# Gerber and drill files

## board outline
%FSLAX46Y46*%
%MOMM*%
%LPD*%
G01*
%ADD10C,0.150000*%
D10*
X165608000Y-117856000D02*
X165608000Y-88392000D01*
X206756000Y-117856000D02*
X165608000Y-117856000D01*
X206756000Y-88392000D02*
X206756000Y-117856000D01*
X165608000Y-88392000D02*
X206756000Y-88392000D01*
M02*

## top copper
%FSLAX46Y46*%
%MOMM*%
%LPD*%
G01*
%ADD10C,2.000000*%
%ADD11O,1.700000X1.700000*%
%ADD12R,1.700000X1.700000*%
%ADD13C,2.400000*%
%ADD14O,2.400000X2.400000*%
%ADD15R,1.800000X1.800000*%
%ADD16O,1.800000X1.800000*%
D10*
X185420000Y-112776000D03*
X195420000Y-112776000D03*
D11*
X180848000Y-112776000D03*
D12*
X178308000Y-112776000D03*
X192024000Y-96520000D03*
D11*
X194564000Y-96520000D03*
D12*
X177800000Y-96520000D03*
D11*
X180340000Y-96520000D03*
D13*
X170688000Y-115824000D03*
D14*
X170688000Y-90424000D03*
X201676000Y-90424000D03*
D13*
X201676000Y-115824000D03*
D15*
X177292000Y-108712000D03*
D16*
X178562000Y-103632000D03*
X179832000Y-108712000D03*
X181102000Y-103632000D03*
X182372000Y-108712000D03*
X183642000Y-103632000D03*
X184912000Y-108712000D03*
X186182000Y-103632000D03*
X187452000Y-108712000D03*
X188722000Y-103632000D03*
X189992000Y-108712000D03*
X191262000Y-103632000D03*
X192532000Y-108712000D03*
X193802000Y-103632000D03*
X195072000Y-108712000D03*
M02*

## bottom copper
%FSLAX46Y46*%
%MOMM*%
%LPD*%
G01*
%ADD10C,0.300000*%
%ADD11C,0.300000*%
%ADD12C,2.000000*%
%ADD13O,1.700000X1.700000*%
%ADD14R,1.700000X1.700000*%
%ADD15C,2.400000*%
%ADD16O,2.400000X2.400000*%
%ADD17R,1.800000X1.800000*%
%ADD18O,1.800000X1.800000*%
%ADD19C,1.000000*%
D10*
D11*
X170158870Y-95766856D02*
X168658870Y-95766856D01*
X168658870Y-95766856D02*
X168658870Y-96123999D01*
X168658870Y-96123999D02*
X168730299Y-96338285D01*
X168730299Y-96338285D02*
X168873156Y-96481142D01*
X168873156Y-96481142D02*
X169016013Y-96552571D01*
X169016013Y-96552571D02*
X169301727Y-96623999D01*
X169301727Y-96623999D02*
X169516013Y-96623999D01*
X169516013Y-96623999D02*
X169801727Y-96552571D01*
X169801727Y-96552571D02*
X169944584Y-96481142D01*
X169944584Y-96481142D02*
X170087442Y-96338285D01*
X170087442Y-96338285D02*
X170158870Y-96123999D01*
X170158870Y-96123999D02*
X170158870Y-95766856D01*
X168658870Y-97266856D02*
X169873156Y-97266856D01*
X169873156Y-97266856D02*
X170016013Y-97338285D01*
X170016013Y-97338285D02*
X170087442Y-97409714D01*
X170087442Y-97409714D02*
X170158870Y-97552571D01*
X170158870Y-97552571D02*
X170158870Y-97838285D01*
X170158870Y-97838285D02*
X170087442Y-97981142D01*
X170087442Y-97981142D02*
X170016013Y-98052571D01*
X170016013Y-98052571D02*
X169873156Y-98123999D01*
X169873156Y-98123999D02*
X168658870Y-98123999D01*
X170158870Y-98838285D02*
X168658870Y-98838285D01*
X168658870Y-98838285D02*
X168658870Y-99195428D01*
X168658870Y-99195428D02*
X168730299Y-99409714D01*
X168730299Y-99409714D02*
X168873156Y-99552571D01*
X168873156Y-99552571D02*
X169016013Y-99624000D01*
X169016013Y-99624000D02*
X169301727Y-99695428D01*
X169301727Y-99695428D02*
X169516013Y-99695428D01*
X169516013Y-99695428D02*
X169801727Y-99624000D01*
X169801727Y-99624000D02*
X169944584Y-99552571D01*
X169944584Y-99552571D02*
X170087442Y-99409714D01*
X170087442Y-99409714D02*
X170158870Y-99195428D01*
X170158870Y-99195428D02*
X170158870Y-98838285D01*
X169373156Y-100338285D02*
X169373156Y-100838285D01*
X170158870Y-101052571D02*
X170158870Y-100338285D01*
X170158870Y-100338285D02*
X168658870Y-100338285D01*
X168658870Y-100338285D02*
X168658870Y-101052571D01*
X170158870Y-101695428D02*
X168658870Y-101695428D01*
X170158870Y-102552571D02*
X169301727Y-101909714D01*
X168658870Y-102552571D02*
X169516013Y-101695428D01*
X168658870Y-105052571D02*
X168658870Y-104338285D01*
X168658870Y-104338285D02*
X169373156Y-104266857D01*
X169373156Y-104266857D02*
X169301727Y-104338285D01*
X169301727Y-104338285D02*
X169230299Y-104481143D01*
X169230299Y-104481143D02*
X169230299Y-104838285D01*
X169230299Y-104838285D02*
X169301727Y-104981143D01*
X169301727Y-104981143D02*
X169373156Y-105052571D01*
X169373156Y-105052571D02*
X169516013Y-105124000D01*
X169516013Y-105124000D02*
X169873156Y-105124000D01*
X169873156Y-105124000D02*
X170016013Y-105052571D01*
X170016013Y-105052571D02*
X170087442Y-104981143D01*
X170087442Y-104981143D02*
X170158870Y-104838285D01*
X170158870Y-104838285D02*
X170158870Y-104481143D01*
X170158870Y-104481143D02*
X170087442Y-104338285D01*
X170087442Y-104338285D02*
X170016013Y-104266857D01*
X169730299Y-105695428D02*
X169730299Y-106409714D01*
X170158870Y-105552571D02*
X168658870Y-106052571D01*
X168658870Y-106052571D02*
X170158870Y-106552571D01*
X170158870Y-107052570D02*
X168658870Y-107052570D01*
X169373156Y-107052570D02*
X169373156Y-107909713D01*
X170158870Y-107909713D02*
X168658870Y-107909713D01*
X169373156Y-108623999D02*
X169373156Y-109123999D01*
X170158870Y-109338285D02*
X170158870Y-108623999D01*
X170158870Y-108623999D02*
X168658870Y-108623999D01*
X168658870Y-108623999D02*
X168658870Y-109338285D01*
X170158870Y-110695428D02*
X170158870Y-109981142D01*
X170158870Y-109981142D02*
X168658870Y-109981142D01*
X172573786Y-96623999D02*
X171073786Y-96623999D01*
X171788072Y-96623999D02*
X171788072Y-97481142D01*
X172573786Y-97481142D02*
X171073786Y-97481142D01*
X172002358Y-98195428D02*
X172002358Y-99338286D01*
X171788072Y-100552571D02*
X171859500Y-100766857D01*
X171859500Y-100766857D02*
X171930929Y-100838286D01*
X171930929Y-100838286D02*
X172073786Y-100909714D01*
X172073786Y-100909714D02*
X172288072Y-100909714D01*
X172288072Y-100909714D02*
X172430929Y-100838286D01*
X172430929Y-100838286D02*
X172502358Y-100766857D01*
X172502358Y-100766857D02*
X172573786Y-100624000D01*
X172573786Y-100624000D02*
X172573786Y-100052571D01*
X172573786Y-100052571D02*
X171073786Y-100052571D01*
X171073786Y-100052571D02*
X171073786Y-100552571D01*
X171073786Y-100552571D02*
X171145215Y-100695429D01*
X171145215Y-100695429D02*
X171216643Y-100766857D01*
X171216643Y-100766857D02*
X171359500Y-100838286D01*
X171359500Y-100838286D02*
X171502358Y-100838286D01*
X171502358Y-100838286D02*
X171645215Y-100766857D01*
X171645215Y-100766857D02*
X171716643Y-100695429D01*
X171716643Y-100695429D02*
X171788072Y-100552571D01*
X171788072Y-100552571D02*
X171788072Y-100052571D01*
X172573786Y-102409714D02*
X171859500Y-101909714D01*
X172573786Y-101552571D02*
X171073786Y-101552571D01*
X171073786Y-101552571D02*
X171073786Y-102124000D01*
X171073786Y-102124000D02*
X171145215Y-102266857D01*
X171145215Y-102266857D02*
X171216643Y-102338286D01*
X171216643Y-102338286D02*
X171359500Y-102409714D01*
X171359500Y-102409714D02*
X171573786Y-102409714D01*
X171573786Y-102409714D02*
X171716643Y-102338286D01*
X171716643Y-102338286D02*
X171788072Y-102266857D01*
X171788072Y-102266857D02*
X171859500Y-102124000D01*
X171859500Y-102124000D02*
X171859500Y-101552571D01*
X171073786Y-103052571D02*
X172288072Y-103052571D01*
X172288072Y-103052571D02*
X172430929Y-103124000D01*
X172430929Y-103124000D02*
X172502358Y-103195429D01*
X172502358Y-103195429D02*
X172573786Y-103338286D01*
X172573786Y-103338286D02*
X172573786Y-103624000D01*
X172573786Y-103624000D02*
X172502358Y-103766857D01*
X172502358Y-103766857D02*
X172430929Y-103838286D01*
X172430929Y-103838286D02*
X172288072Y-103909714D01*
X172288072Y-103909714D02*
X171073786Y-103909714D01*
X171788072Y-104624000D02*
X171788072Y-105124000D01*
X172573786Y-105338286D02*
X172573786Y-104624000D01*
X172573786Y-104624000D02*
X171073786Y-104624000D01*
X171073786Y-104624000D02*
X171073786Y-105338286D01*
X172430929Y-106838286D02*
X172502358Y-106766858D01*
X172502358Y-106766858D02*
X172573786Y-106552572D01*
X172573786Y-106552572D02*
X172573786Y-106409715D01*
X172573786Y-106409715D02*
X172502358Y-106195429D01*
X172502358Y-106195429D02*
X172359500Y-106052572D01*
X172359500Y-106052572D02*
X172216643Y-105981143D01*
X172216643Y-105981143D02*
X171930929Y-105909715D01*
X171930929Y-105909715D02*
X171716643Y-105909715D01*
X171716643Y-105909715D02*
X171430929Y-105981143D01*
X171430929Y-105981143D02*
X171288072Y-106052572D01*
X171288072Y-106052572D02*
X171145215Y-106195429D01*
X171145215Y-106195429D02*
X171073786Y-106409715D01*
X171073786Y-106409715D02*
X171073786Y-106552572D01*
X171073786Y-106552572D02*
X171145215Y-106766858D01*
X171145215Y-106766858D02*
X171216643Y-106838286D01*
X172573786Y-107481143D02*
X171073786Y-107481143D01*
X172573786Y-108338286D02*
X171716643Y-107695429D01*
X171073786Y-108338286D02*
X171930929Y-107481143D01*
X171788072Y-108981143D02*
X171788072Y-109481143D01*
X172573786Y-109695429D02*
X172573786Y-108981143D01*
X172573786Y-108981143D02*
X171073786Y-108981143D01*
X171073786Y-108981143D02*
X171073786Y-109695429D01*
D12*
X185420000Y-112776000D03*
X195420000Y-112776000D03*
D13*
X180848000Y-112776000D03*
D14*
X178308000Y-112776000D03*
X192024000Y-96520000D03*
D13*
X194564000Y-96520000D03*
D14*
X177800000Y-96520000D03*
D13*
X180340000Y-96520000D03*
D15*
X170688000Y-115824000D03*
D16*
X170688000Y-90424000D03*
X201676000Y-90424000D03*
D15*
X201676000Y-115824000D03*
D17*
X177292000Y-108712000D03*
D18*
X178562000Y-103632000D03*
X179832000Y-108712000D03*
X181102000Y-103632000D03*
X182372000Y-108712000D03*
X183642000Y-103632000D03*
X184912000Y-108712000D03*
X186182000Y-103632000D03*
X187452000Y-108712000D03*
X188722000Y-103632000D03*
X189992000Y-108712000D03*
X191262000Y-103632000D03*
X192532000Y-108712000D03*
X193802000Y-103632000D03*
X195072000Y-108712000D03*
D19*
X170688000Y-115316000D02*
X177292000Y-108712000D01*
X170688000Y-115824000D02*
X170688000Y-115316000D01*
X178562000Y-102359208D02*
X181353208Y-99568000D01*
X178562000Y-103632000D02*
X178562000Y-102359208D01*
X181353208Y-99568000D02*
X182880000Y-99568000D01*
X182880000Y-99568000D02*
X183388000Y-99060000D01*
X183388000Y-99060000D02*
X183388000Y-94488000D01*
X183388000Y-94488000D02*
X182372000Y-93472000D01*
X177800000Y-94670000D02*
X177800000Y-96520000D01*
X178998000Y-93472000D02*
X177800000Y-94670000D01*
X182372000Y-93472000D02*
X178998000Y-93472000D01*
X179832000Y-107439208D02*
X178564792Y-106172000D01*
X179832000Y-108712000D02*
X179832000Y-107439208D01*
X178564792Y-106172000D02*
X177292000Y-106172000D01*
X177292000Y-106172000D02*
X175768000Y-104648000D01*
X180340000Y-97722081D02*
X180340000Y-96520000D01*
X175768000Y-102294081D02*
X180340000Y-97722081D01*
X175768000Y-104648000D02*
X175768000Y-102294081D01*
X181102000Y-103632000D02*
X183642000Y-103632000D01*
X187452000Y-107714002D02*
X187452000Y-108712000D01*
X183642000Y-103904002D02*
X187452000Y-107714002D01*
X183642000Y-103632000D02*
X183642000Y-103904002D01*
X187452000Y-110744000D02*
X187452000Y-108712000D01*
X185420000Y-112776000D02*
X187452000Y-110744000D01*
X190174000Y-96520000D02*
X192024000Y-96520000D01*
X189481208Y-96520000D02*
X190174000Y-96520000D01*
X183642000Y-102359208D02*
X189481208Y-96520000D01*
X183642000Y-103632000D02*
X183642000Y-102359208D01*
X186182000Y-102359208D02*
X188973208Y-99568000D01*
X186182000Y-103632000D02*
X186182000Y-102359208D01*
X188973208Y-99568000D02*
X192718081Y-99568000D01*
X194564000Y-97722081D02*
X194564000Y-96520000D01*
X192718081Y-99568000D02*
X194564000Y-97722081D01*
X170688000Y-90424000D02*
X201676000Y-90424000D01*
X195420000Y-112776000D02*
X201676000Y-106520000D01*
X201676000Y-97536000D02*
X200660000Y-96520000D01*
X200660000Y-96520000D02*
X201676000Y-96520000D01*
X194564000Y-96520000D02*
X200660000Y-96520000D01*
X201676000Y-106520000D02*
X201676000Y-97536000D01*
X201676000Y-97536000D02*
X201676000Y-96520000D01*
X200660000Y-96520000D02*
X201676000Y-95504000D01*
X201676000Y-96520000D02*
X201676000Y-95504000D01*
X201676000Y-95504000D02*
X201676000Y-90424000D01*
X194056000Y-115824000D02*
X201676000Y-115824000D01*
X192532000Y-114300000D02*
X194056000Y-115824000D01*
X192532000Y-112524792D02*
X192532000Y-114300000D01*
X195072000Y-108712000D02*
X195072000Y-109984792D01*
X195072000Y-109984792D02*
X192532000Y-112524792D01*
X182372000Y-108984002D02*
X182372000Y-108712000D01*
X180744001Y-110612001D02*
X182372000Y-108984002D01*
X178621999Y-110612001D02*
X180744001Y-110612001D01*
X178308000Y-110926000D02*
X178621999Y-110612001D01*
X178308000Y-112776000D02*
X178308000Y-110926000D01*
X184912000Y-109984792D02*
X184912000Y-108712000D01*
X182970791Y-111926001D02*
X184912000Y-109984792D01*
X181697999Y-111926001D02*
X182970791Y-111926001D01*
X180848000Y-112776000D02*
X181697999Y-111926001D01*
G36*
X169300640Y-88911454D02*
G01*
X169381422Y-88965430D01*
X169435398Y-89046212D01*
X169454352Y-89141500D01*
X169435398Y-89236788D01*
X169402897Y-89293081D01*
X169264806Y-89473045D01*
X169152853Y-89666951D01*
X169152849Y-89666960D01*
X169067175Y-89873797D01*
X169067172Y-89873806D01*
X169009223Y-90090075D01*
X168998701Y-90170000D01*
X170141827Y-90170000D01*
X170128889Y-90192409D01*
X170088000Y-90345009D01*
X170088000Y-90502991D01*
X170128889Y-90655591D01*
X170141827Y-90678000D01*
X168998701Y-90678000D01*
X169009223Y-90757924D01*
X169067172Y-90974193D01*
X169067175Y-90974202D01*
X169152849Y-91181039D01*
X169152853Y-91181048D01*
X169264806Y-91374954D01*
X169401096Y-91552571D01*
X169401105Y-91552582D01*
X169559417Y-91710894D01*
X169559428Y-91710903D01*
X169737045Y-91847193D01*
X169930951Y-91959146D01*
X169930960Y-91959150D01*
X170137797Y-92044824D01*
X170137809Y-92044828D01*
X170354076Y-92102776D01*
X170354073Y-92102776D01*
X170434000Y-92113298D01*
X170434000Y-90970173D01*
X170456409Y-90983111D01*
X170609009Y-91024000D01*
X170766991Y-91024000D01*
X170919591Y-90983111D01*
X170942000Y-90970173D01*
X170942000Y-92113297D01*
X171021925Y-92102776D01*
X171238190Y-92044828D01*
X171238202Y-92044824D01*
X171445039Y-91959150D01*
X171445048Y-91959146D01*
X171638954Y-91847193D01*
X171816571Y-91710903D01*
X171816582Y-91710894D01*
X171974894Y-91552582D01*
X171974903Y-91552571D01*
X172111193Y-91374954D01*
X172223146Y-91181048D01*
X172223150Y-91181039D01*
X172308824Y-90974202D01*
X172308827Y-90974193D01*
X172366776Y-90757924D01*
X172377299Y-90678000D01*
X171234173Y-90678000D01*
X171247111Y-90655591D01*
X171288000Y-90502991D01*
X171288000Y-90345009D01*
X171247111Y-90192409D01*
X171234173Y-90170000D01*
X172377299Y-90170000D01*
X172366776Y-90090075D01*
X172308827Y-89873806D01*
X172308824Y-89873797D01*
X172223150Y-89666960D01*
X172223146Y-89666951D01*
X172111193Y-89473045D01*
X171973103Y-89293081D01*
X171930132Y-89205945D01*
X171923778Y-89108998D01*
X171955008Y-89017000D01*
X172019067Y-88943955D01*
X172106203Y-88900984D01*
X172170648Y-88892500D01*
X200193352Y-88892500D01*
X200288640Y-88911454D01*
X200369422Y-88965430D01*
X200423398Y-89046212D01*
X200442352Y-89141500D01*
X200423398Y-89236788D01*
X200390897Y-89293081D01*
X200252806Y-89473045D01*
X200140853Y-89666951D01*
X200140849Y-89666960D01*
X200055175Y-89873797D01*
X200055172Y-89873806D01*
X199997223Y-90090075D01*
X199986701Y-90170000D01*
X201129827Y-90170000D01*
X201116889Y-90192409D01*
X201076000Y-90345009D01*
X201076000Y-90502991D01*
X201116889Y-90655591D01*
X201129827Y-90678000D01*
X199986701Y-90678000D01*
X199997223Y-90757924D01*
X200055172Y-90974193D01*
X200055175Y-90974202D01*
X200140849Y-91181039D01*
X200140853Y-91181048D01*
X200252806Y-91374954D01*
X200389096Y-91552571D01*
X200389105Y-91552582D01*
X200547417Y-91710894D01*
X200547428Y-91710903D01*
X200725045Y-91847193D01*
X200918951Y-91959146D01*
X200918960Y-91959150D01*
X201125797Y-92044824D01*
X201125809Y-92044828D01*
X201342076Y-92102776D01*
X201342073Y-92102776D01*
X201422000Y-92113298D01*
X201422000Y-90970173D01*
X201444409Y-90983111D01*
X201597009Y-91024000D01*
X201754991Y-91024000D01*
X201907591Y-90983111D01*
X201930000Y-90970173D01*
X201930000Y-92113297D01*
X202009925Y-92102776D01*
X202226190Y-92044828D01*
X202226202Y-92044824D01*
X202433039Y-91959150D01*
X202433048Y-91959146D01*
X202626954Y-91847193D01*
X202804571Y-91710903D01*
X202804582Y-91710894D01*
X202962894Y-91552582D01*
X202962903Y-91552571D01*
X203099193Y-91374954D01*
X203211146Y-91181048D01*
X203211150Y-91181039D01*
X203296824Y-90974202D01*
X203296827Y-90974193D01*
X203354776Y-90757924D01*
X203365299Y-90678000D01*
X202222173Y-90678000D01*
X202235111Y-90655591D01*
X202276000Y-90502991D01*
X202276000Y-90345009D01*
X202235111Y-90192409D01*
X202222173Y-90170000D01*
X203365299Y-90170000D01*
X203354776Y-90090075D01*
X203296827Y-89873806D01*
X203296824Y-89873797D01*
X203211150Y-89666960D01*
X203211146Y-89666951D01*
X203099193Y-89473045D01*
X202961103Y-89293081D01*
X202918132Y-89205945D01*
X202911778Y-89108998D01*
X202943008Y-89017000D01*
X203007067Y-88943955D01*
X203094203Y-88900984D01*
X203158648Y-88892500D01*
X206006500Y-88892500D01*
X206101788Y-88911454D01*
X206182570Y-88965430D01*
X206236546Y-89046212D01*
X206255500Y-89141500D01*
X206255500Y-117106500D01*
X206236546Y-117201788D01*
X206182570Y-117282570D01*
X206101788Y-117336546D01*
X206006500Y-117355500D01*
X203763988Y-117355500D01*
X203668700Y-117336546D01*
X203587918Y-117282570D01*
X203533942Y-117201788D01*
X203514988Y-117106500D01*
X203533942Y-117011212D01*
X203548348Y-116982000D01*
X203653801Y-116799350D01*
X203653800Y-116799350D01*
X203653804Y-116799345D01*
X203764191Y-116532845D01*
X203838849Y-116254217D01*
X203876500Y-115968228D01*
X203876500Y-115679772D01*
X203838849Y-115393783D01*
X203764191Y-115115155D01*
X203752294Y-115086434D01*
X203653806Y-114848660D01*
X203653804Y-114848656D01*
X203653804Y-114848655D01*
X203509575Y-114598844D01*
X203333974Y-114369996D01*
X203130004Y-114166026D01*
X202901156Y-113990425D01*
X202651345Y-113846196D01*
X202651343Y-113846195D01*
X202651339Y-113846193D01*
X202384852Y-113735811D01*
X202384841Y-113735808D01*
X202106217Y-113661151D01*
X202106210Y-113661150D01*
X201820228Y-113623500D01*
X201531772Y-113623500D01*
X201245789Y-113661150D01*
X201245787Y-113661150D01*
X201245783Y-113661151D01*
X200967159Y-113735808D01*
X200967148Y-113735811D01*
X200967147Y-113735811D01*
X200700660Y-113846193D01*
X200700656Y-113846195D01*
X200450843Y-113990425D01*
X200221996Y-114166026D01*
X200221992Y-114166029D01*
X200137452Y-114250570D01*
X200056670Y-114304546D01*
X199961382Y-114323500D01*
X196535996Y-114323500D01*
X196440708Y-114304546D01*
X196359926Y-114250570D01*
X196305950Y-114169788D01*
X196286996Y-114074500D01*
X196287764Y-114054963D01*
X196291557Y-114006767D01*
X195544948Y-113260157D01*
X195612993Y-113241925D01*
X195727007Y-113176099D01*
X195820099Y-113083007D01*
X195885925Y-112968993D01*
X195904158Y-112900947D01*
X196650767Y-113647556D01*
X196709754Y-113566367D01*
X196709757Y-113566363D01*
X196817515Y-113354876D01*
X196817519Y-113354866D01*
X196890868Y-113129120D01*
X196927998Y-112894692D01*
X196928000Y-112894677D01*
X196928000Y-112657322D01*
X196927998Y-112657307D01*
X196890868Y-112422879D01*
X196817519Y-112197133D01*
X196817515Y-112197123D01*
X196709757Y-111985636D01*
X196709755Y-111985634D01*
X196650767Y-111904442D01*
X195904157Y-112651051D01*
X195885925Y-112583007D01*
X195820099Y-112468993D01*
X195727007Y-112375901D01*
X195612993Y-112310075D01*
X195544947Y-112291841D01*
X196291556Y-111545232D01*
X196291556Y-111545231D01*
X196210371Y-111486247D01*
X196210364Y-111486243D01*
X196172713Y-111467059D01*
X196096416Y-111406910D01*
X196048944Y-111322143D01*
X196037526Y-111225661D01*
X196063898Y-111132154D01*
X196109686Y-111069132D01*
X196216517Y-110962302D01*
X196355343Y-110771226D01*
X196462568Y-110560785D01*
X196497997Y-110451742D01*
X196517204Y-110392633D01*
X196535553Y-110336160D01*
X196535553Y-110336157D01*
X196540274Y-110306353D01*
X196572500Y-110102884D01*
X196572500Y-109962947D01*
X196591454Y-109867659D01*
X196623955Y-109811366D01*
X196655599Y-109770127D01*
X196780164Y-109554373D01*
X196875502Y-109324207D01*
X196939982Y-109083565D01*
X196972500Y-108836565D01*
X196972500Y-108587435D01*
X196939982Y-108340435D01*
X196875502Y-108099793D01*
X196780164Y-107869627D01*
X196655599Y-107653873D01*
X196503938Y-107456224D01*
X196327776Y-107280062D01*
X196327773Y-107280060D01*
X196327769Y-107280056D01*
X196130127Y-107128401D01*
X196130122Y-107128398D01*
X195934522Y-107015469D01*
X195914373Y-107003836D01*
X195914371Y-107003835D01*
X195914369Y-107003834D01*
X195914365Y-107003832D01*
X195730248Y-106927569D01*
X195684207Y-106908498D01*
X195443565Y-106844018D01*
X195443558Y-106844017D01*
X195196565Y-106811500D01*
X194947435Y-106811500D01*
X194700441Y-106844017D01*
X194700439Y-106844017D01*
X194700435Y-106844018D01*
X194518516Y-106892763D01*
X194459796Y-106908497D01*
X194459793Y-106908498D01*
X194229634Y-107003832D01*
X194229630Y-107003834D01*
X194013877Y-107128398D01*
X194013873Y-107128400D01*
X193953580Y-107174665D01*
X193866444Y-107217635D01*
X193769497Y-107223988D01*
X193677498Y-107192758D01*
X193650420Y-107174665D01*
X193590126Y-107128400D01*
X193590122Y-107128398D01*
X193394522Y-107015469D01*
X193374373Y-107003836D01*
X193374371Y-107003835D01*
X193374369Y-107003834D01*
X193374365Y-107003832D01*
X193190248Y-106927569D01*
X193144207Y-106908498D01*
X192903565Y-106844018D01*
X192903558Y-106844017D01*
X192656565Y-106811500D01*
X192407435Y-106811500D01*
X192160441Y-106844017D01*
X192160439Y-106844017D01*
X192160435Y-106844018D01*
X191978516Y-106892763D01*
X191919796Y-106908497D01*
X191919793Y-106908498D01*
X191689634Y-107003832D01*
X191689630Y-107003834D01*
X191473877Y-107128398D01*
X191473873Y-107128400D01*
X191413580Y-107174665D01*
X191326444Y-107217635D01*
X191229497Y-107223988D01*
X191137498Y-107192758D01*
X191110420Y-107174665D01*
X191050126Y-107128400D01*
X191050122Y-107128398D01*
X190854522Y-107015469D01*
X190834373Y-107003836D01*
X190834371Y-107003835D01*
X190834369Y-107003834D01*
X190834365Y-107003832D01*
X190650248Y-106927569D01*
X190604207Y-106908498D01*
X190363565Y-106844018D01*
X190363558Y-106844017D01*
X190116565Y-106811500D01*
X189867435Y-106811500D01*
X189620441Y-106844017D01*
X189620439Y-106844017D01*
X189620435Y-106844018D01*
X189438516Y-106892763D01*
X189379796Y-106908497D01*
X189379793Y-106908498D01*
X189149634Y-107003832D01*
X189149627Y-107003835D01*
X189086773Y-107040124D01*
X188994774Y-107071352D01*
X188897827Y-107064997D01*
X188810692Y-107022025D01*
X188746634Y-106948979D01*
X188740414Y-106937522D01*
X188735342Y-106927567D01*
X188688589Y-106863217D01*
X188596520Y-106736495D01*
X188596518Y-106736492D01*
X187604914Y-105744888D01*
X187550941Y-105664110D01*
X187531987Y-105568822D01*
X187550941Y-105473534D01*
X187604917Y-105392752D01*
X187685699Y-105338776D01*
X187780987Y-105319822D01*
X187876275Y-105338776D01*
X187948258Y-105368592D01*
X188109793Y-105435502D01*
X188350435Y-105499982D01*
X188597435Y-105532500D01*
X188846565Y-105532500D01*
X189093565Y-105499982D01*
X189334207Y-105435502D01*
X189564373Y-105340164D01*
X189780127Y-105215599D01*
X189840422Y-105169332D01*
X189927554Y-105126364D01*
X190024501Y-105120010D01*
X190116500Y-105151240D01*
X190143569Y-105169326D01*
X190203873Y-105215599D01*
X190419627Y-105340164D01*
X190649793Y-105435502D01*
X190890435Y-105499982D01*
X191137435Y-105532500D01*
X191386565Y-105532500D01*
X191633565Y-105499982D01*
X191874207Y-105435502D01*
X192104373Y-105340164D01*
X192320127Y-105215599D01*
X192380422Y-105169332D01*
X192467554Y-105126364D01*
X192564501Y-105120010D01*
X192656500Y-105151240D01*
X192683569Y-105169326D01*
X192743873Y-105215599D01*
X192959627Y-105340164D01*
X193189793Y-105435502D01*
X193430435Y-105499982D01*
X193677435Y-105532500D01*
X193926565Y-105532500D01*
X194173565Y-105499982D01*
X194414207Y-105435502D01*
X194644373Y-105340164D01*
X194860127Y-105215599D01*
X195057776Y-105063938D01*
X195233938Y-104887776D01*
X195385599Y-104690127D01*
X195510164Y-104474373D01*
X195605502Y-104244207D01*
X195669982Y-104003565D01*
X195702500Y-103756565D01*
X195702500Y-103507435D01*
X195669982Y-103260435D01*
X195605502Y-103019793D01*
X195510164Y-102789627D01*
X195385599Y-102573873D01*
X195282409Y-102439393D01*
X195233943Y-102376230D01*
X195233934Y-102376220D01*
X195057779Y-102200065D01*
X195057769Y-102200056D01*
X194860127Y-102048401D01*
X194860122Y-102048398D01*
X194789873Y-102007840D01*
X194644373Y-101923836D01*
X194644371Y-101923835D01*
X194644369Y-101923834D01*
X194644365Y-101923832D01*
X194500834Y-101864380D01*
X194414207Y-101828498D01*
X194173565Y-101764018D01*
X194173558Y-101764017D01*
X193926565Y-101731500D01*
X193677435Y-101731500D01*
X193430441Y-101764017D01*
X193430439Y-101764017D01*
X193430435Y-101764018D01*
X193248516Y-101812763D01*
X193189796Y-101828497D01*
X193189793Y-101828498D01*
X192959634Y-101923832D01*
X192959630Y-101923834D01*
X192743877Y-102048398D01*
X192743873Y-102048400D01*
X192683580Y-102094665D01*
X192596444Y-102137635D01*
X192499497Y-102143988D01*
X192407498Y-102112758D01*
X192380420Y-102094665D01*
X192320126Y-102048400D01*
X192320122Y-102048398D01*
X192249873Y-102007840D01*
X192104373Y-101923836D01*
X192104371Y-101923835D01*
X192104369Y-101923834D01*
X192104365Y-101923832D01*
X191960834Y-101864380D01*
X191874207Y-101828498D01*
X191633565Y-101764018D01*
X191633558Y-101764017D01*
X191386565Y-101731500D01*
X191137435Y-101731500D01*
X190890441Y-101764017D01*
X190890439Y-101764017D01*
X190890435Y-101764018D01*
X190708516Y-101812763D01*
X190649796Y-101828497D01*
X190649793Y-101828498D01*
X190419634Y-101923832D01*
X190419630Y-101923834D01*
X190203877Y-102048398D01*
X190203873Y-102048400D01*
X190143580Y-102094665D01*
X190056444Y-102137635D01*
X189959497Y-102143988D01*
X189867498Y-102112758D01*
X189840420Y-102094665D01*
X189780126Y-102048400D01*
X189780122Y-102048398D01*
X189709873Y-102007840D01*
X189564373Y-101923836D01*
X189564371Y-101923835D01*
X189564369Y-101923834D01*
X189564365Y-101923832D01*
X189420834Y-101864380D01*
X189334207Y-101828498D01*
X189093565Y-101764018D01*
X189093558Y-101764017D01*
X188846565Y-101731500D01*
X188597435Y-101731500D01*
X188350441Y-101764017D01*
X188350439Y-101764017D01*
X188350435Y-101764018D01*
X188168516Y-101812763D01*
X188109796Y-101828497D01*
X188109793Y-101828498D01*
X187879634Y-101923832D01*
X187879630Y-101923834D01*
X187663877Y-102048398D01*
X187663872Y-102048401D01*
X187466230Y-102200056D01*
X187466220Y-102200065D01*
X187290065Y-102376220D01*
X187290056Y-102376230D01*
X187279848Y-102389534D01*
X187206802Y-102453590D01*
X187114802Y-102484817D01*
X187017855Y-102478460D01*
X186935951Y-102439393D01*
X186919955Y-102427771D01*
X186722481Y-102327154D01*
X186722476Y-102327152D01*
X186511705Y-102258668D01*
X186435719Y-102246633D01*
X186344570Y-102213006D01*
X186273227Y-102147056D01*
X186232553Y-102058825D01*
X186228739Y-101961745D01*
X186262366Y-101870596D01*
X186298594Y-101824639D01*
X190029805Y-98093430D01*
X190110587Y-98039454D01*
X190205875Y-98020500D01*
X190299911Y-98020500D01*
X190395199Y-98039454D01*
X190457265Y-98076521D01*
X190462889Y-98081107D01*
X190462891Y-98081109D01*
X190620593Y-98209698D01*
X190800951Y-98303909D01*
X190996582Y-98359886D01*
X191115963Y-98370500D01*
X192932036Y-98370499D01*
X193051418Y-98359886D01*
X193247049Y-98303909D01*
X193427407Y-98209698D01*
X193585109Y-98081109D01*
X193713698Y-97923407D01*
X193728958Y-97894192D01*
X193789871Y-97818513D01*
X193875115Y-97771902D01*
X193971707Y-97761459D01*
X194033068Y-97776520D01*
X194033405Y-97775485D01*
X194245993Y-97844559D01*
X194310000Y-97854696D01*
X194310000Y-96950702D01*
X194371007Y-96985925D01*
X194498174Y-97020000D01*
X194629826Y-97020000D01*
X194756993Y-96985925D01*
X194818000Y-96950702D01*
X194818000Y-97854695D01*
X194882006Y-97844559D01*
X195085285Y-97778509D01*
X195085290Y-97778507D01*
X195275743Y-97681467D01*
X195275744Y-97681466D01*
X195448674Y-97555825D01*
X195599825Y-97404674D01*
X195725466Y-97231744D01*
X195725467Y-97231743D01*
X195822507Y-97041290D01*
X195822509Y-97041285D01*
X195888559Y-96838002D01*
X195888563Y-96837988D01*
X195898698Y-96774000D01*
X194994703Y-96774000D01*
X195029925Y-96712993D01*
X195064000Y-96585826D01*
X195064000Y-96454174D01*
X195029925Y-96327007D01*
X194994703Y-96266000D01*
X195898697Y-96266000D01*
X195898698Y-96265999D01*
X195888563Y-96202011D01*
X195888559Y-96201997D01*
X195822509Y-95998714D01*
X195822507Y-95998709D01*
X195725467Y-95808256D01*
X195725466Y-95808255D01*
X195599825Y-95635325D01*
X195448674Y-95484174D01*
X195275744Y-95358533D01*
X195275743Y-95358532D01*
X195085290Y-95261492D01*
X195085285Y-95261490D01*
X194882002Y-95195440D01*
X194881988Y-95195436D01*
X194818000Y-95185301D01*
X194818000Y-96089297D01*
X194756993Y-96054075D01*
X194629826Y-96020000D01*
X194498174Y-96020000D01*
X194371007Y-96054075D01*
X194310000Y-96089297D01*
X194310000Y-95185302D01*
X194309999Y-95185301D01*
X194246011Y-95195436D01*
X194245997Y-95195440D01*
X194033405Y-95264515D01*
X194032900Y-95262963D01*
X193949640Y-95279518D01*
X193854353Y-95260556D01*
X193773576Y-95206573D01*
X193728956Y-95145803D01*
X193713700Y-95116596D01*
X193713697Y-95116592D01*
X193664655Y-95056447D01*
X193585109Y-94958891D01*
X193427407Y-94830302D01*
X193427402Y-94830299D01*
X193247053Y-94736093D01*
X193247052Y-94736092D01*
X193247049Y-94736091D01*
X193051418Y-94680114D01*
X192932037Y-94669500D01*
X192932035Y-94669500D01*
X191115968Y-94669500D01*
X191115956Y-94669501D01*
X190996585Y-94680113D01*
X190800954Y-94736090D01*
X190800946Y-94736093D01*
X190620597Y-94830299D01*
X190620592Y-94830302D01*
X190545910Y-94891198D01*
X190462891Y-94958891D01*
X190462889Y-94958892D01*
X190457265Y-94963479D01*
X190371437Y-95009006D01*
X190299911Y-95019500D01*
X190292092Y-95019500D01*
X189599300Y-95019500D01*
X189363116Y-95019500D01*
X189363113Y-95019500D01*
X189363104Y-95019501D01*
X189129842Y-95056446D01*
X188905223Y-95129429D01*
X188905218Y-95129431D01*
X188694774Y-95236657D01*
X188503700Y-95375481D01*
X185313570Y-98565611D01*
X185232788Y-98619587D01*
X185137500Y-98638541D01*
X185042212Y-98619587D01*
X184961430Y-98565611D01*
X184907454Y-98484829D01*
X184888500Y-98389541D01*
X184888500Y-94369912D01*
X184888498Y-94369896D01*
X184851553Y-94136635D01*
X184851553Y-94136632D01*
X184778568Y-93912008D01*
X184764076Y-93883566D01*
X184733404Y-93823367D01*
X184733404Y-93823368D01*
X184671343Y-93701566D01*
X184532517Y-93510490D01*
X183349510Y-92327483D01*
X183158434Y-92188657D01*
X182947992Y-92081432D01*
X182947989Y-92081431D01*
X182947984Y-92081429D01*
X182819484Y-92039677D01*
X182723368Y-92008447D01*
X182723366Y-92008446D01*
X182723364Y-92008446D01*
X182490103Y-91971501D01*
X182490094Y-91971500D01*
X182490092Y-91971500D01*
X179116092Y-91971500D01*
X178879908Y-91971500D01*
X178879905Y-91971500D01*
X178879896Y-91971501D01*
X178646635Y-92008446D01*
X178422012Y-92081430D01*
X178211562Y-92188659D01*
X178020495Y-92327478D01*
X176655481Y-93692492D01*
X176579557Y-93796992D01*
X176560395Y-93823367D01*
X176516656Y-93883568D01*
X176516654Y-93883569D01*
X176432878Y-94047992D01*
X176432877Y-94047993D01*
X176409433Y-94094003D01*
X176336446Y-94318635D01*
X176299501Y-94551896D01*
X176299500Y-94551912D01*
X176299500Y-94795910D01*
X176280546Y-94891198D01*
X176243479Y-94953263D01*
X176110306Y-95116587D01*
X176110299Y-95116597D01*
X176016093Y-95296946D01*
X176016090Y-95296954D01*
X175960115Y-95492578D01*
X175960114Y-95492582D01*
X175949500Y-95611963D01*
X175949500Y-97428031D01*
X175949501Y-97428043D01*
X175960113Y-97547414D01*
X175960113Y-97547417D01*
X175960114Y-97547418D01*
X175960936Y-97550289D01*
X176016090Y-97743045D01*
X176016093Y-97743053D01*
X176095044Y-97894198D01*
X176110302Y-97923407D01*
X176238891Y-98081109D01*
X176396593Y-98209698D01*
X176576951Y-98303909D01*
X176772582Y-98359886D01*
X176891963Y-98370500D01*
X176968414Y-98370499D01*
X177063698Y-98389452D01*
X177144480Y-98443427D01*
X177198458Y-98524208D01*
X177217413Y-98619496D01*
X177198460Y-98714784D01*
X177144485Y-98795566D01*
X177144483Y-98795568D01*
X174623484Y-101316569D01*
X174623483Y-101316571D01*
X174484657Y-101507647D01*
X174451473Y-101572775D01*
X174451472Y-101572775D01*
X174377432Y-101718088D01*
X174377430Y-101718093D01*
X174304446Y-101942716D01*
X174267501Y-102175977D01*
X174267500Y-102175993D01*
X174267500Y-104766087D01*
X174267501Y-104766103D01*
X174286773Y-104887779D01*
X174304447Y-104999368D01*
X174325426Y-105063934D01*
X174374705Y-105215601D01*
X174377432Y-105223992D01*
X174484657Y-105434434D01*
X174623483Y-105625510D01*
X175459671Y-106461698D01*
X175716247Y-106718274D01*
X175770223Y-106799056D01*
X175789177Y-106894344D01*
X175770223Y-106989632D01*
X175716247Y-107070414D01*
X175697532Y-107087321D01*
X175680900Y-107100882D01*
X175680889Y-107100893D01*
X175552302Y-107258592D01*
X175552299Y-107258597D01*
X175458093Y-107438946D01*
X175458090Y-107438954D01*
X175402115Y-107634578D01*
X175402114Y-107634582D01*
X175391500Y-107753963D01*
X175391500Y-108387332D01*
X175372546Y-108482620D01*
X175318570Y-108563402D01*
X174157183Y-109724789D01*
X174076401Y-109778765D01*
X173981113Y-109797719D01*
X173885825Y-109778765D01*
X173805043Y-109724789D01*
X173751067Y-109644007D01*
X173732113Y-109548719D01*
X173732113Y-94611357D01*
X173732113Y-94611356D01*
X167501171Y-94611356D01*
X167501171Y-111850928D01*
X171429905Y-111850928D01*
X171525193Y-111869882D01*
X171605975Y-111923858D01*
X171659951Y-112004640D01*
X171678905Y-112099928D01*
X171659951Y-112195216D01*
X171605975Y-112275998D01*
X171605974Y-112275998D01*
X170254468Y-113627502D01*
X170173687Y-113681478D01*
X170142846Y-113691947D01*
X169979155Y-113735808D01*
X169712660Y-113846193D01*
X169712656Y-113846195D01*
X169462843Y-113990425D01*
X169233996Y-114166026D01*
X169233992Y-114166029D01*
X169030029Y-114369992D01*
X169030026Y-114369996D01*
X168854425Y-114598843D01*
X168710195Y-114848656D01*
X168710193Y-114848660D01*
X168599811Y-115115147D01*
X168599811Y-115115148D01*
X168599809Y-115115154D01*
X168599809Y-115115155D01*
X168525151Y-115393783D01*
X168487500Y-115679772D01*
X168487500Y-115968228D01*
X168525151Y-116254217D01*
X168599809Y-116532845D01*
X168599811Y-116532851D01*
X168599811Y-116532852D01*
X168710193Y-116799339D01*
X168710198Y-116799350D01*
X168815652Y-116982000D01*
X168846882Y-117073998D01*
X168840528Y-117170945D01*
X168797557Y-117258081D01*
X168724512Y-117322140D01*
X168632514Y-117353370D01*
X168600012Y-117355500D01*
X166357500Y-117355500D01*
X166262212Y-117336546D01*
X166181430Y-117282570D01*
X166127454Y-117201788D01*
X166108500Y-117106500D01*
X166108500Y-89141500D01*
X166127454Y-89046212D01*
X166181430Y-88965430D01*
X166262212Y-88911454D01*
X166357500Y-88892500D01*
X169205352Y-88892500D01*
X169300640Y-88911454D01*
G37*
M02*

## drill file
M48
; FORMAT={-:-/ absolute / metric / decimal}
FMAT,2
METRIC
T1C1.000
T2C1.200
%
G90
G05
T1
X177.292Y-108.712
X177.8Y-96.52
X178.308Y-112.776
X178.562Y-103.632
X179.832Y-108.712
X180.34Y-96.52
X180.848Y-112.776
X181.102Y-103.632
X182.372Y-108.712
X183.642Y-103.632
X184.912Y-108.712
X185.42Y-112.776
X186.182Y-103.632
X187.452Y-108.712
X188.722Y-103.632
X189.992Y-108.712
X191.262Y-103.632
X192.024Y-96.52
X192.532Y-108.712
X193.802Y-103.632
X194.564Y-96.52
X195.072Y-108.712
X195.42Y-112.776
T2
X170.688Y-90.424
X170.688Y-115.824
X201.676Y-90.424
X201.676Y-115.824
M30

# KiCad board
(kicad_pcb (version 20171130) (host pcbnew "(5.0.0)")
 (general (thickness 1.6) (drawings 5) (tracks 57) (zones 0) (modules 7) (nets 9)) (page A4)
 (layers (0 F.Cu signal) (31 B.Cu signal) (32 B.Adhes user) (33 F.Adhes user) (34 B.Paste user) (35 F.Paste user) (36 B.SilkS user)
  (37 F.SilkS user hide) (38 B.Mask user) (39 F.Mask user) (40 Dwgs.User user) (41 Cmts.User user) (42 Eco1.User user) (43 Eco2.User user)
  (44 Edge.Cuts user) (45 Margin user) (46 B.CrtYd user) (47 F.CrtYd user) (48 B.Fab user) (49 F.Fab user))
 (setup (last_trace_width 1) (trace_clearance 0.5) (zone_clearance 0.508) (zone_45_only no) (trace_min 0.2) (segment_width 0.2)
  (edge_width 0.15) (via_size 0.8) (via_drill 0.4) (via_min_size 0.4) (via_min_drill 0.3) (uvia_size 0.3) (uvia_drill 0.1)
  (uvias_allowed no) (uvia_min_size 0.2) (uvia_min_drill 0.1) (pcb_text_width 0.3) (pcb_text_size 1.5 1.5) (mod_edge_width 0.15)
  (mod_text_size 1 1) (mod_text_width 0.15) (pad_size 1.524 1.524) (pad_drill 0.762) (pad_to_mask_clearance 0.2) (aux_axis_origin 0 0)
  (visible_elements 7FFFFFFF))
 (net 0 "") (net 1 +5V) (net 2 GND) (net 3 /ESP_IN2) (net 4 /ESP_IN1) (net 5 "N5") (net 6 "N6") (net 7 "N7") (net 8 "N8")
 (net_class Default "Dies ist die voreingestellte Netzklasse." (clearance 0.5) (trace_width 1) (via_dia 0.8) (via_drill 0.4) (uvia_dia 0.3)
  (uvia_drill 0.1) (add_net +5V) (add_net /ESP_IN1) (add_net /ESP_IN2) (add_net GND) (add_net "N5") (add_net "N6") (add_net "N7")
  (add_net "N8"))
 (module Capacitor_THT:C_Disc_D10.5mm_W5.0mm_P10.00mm (layer F.Cu) (at 185.42 112.776)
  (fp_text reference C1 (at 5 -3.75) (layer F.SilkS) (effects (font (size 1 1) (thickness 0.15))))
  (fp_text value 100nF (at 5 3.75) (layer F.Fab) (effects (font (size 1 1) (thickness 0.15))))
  (pad 1 thru_hole circle (at 0 0) (size 2 2) (drill 1) (layers *.Cu *.Mask) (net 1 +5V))
  (pad 2 thru_hole circle (at 10 0) (size 2 2) (drill 1) (layers *.Cu *.Mask) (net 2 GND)))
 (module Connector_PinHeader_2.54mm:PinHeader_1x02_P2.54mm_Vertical (layer F.Cu) (at 178.308 112.776 90)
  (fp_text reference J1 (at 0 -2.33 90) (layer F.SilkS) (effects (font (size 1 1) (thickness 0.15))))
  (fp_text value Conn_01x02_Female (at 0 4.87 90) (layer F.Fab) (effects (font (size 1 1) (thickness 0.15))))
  (pad 2 thru_hole oval (at 0 2.54 90) (size 1.7 1.7) (drill 1) (layers *.Cu *.Mask) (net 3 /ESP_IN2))
  (pad 1 thru_hole rect (at 0 0 90) (size 1.7 1.7) (drill 1) (layers *.Cu *.Mask) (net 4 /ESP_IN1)))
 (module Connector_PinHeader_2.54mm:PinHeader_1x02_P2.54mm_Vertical (layer F.Cu) (at 192.024 96.52 90)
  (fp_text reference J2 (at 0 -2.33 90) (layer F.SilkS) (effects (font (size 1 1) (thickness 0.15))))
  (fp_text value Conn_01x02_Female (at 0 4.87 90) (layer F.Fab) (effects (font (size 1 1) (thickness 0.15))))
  (pad 1 thru_hole rect (at 0 0 90) (size 1.7 1.7) (drill 1) (layers *.Cu *.Mask) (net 1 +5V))
  (pad 2 thru_hole oval (at 0 2.54 90) (size 1.7 1.7) (drill 1) (layers *.Cu *.Mask) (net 2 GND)))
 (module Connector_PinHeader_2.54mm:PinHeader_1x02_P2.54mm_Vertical (layer F.Cu) (at 177.8 96.52 90)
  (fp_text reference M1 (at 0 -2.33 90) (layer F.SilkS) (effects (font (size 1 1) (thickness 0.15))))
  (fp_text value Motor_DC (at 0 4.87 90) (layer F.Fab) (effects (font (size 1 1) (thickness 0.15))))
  (pad 1 thru_hole rect (at 0 0 90) (size 1.7 1.7) (drill 1) (layers *.Cu *.Mask) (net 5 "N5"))
  (pad 2 thru_hole oval (at 0 2.54 90) (size 1.7 1.7) (drill 1) (layers *.Cu *.Mask) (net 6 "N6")))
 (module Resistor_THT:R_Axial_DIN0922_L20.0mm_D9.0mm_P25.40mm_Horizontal (layer F.Cu) (at 170.688 115.824 90)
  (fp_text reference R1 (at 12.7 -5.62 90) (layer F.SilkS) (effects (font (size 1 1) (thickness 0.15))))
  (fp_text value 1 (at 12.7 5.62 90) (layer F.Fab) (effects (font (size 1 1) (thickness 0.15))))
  (pad 1 thru_hole circle (at 0 0 90) (size 2.4 2.4) (drill 1.2) (layers *.Cu *.Mask) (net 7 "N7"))
  (pad 2 thru_hole oval (at 25.4 0 90) (size 2.4 2.4) (drill 1.2) (layers *.Cu *.Mask) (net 2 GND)))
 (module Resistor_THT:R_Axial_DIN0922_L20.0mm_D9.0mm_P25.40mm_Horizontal (layer F.Cu) (at 201.676 115.824 90)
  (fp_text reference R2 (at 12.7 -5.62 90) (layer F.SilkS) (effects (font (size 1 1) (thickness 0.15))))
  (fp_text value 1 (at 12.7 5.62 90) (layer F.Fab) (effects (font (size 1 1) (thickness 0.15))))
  (pad 2 thru_hole oval (at 25.4 0 90) (size 2.4 2.4) (drill 1.2) (layers *.Cu *.Mask) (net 2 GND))
  (pad 1 thru_hole circle (at 0 0 90) (size 2.4 2.4) (drill 1.2) (layers *.Cu *.Mask) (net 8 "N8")))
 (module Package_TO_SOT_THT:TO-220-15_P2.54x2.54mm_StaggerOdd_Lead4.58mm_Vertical (layer F.Cu) (at 177.292 108.712)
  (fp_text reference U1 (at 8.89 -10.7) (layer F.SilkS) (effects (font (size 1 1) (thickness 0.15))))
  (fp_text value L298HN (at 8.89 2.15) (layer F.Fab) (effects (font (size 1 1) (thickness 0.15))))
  (pad 1 thru_hole rect (at 0 0) (size 1.8 1.8) (drill 1) (layers *.Cu *.Mask) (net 7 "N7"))
  (pad 2 thru_hole oval (at 1.27 -5.08) (size 1.8 1.8) (drill 1) (layers *.Cu *.Mask) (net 5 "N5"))
  (pad 3 thru_hole oval (at 2.54 0) (size 1.8 1.8) (drill 1) (layers *.Cu *.Mask) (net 6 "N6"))
  (pad 4 thru_hole oval (at 3.81 -5.08) (size 1.8 1.8) (drill 1) (layers *.Cu *.Mask) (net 1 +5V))
  (pad 5 thru_hole oval (at 5.08 0) (size 1.8 1.8) (drill 1) (layers *.Cu *.Mask) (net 4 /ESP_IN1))
  (pad 6 thru_hole oval (at 6.35 -5.08) (size 1.8 1.8) (drill 1) (layers *.Cu *.Mask) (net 1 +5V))
  (pad 7 thru_hole oval (at 7.62 0) (size 1.8 1.8) (drill 1) (layers *.Cu *.Mask) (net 3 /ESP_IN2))
  (pad 8 thru_hole oval (at 8.89 -5.08) (size 1.8 1.8) (drill 1) (layers *.Cu *.Mask) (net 2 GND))
  (pad 9 thru_hole oval (at 10.16 0) (size 1.8 1.8) (drill 1) (layers *.Cu *.Mask) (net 1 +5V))
  (pad 10 thru_hole oval (at 11.43 -5.08) (size 1.8 1.8) (drill 1) (layers *.Cu *.Mask))
  (pad 11 thru_hole oval (at 12.7 0) (size 1.8 1.8) (drill 1) (layers *.Cu *.Mask))
  (pad 12 thru_hole oval (at 13.97 -5.08) (size 1.8 1.8) (drill 1) (layers *.Cu *.Mask))
  (pad 13 thru_hole oval (at 15.24 0) (size 1.8 1.8) (drill 1) (layers *.Cu *.Mask))
  (pad 14 thru_hole oval (at 16.51 -5.08) (size 1.8 1.8) (drill 1) (layers *.Cu *.Mask))
  (pad 15 thru_hole oval (at 17.78 0) (size 1.8 1.8) (drill 1) (layers *.Cu *.Mask) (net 8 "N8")))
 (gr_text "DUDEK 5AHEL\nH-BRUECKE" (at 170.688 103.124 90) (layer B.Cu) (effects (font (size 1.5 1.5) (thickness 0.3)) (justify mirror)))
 (gr_line (start 165.608 117.856) (end 165.608 88.392) (layer Edge.Cuts) (width 0.15))
 (gr_line (start 206.756 117.856) (end 165.608 117.856) (layer Edge.Cuts) (width 0.15))
 (gr_line (start 206.756 88.392) (end 206.756 117.856) (layer Edge.Cuts) (width 0.15))
 (gr_line (start 165.608 88.392) (end 206.756 88.392) (layer Edge.Cuts) (width 0.15))
 (segment (start 170.688 115.316) (end 177.292 108.712) (width 1) (layer B.Cu) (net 7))
 (segment (start 170.688 115.824) (end 170.688 115.316) (width 1) (layer B.Cu) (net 7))
 (segment (start 178.562 102.359208) (end 181.353208 99.568) (width 1) (layer B.Cu) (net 5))
 (segment (start 178.562 103.632) (end 178.562 102.359208) (width 1) (layer B.Cu) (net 5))
 (segment (start 181.353208 99.568) (end 182.88 99.568) (width 1) (layer B.Cu) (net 5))
 (segment (start 182.88 99.568) (end 183.388 99.06) (width 1) (layer B.Cu) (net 5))
 (segment (start 183.388 99.06) (end 183.388 94.488) (width 1) (layer B.Cu) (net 5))
 (segment (start 183.388 94.488) (end 182.372 93.472) (width 1) (layer B.Cu) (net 5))
 (segment (start 177.8 94.67) (end 177.8 96.52) (width 1) (layer B.Cu) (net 5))
 (segment (start 178.998 93.472) (end 177.8 94.67) (width 1) (layer B.Cu) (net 5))
 (segment (start 182.372 93.472) (end 178.998 93.472) (width 1) (layer B.Cu) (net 5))
 (segment (start 179.832 107.439208) (end 178.564792 106.172) (width 1) (layer B.Cu) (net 6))
 (segment (start 179.832 108.712) (end 179.832 107.439208) (width 1) (layer B.Cu) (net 6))
 (segment (start 178.564792 106.172) (end 177.292 106.172) (width 1) (layer B.Cu) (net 6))
 (segment (start 177.292 106.172) (end 175.768 104.648) (width 1) (layer B.Cu) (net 6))
 (segment (start 180.34 97.722081) (end 180.34 96.52) (width 1) (layer B.Cu) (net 6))
 (segment (start 175.768 102.294081) (end 180.34 97.722081) (width 1) (layer B.Cu) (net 6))
 (segment (start 175.768 104.648) (end 175.768 102.294081) (width 1) (layer B.Cu) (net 6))
 (segment (start 181.102 103.632) (end 183.642 103.632) (width 1) (layer B.Cu) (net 1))
 (segment (start 187.452 107.714002) (end 187.452 108.712) (width 1) (layer B.Cu) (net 1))
 (segment (start 183.642 103.904002) (end 187.452 107.714002) (width 1) (layer B.Cu) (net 1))
 (segment (start 183.642 103.632) (end 183.642 103.904002) (width 1) (layer B.Cu) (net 1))
 (segment (start 187.452 110.744) (end 187.452 108.712) (width 1) (layer B.Cu) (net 1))
 (segment (start 185.42 112.776) (end 187.452 110.744) (width 1) (layer B.Cu) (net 1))
 (segment (start 190.174 96.52) (end 192.024 96.52) (width 1) (layer B.Cu) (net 1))
 (segment (start 189.481208 96.52) (end 190.174 96.52) (width 1) (layer B.Cu) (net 1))
 (segment (start 183.642 102.359208) (end 189.481208 96.52) (width 1) (layer B.Cu) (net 1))
 (segment (start 183.642 103.632) (end 183.642 102.359208) (width 1) (layer B.Cu) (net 1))
 (segment (start 186.182 102.359208) (end 188.973208 99.568) (width 1) (layer B.Cu) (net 2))
 (segment (start 186.182 103.632) (end 186.182 102.359208) (width 1) (layer B.Cu) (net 2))
 (segment (start 188.973208 99.568) (end 192.718081 99.568) (width 1) (layer B.Cu) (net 2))
 (segment (start 194.564 97.722081) (end 194.564 96.52) (width 1) (layer B.Cu) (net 2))
 (segment (start 192.718081 99.568) (end 194.564 97.722081) (width 1) (layer B.Cu) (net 2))
 (segment (start 170.688 90.424) (end 201.676 90.424) (width 1) (layer B.Cu) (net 2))
 (segment (start 195.42 112.776) (end 201.676 106.52) (width 1) (layer B.Cu) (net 2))
 (segment (start 201.676 97.536) (end 200.66 96.52) (width 1) (layer B.Cu) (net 2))
 (segment (start 200.66 96.52) (end 201.676 96.52) (width 1) (layer B.Cu) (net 2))
 (segment (start 194.564 96.52) (end 200.66 96.52) (width 1) (layer B.Cu) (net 2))
 (segment (start 201.676 106.52) (end 201.676 97.536) (width 1) (layer B.Cu) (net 2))
 (segment (start 201.676 97.536) (end 201.676 96.52) (width 1) (layer B.Cu) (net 2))
 (segment (start 200.66 96.52) (end 201.676 95.504) (width 1) (layer B.Cu) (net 2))
 (segment (start 201.676 96.52) (end 201.676 95.504) (width 1) (layer B.Cu) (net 2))
 (segment (start 201.676 95.504) (end 201.676 90.424) (width 1) (layer B.Cu) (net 2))
 (segment (start 194.056 115.824) (end 201.676 115.824) (width 1) (layer B.Cu) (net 8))
 (segment (start 192.532 114.3) (end 194.056 115.824) (width 1) (layer B.Cu) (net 8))
 (segment (start 192.532 112.524792) (end 192.532 114.3) (width 1) (layer B.Cu) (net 8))
 (segment (start 195.072 108.712) (end 195.072 109.984792) (width 1) (layer B.Cu) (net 8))
 (segment (start 195.072 109.984792) (end 192.532 112.524792) (width 1) (layer B.Cu) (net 8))
 (segment (start 182.372 108.984002) (end 182.372 108.712) (width 1) (layer B.Cu) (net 4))
 (segment (start 180.744001 110.612001) (end 182.372 108.984002) (width 1) (layer B.Cu) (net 4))
 (segment (start 178.621999 110.612001) (end 180.744001 110.612001) (width 1) (layer B.Cu) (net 4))
 (segment (start 178.308 110.926) (end 178.621999 110.612001) (width 1) (layer B.Cu) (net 4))
 (segment (start 178.308 112.776) (end 178.308 110.926) (width 1) (layer B.Cu) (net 4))
 (segment (start 184.912 109.984792) (end 184.912 108.712) (width 1) (layer B.Cu) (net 3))
 (segment (start 182.970791 111.926001) (end 184.912 109.984792) (width 1) (layer B.Cu) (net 3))
 (segment (start 181.697999 111.926001) (end 182.970791 111.926001) (width 1) (layer B.Cu) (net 3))
 (segment (start 180.848 112.776) (end 181.697999 111.926001) (width 1) (layer B.Cu) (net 3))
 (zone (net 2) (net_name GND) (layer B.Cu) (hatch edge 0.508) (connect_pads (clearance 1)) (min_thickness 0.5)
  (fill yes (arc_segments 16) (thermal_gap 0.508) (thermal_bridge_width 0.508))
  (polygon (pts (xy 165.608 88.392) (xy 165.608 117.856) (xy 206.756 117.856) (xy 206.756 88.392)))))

